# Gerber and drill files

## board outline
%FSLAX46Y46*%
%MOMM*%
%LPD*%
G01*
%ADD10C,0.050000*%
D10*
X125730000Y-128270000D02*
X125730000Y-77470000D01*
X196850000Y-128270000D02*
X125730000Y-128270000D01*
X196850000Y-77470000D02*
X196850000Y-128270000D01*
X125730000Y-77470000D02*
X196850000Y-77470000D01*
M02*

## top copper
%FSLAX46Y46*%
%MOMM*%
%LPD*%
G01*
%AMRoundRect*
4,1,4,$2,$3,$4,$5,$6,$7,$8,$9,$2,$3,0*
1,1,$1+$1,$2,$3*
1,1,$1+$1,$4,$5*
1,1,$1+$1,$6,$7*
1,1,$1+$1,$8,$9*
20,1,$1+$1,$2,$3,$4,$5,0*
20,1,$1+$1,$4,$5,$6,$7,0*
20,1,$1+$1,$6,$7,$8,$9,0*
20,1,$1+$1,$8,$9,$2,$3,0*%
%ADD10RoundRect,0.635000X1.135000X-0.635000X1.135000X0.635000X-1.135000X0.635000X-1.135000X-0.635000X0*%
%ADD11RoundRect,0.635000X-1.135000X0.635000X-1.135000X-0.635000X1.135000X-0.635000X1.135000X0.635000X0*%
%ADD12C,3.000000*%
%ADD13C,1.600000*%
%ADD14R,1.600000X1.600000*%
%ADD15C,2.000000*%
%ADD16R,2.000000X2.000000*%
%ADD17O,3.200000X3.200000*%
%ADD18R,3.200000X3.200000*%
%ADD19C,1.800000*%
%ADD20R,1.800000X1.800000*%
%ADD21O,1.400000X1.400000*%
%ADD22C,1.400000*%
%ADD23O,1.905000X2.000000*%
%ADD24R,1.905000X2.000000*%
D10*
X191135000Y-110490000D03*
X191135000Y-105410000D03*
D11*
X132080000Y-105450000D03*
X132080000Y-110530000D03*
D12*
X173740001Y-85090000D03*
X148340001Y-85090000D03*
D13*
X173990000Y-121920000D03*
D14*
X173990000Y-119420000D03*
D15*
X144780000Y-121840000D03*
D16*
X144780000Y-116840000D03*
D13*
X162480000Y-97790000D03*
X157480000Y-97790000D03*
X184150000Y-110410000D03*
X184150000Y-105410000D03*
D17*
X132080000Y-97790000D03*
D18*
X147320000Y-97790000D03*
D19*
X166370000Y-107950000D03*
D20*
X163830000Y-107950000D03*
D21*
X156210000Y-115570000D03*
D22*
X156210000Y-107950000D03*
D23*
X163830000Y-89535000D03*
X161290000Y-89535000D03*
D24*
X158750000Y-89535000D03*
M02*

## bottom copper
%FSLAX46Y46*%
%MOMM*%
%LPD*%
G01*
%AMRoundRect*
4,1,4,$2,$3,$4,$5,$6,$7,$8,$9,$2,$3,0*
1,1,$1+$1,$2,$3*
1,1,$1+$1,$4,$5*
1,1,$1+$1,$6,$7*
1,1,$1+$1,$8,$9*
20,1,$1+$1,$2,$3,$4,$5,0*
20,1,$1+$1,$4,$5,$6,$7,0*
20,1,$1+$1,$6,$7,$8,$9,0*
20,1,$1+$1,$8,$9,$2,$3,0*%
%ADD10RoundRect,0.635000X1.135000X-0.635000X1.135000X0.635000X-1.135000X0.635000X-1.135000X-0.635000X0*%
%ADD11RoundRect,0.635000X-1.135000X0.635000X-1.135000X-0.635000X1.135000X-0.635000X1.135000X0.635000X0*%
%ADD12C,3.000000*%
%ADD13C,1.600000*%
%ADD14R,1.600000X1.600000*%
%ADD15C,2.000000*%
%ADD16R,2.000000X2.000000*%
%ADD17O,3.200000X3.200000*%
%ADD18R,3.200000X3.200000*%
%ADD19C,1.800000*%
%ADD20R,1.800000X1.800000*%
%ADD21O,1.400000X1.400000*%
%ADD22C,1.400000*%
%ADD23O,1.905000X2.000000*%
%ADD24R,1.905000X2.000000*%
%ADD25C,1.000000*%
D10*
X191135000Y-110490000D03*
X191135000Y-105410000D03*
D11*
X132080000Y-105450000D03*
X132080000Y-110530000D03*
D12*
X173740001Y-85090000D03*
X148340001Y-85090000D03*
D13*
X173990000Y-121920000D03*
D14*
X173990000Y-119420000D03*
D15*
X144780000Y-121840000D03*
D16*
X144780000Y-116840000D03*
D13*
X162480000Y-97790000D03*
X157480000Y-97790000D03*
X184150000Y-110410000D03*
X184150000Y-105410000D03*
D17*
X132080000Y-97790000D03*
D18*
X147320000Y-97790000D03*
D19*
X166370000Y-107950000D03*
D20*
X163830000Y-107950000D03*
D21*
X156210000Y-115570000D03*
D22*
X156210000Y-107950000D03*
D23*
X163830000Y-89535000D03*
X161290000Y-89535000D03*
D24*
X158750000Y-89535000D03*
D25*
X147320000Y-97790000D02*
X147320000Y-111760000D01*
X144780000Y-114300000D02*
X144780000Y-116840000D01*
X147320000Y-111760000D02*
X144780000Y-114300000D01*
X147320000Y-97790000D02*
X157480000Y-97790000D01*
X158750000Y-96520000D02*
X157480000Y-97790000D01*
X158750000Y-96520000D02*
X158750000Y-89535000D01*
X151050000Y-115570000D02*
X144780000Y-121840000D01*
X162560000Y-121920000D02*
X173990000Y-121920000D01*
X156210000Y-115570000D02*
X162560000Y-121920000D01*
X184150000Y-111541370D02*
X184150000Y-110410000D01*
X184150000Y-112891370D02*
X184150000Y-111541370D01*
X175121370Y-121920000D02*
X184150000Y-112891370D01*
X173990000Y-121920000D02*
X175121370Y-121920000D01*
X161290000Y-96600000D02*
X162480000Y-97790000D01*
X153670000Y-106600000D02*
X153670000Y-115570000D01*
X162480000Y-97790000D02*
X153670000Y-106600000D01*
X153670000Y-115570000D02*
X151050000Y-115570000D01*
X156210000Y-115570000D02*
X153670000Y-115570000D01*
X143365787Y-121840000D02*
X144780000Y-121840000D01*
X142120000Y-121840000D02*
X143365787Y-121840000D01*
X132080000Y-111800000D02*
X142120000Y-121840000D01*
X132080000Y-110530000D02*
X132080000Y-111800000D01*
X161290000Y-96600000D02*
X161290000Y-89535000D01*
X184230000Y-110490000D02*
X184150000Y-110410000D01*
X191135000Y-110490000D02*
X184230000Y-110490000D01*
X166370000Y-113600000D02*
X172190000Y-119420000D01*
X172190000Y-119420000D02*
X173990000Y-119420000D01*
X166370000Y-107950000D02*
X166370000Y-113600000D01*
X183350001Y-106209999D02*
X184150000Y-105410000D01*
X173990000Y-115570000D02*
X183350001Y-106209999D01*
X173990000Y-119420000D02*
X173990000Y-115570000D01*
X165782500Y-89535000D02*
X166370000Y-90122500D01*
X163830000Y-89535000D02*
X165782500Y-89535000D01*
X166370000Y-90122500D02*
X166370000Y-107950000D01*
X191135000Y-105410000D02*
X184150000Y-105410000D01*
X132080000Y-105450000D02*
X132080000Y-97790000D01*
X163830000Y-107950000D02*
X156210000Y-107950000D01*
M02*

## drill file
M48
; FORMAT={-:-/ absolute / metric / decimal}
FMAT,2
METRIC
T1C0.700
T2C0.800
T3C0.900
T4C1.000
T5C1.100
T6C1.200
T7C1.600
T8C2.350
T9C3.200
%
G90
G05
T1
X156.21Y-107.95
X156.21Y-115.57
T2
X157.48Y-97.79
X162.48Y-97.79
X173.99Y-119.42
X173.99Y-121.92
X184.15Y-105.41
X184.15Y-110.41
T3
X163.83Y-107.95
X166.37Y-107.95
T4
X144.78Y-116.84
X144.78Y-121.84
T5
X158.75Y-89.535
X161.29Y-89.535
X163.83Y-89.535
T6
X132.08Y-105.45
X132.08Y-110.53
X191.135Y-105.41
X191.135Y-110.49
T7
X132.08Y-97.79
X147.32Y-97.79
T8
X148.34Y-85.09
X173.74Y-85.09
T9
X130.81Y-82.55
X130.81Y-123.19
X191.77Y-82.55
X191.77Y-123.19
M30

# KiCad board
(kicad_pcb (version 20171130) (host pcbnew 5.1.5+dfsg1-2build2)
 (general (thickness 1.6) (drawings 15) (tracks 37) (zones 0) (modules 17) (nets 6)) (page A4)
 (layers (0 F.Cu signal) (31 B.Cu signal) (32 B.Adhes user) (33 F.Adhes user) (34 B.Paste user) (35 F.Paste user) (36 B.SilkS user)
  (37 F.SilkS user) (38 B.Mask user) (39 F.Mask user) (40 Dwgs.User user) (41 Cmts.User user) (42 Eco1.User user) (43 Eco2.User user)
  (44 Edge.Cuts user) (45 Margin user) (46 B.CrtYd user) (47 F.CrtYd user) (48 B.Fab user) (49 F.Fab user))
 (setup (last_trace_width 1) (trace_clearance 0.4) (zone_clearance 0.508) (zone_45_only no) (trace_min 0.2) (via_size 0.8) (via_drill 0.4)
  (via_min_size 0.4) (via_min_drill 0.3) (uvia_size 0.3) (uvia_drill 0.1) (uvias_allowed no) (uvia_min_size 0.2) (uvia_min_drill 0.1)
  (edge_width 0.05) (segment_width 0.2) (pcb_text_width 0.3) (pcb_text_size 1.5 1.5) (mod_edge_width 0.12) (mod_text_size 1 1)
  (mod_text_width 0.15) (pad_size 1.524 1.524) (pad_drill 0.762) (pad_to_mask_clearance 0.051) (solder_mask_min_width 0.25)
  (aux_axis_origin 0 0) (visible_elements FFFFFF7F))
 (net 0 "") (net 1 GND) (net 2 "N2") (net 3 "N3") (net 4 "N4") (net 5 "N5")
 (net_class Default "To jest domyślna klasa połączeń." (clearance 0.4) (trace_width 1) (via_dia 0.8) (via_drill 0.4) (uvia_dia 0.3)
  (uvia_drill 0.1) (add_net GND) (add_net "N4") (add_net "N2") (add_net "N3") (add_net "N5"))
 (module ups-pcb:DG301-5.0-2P (layer F.Cu) (at 191.135 107.99 90)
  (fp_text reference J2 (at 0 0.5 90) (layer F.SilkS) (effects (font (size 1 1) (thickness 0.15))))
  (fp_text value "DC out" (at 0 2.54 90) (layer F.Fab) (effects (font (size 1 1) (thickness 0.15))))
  (pad 1 thru_hole roundrect (at -2.5 0 90) (size 2.54 3.54) (drill 1.2) (layers *.Cu *.Mask) (roundrect_rratio 0.25) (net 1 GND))
  (pad 2 thru_hole roundrect (at 2.58 0 90) (size 2.54 3.54) (drill 1.2) (layers *.Cu *.Mask) (roundrect_rratio 0.25) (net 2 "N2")))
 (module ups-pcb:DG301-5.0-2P (layer F.Cu) (at 132.08 107.95 270)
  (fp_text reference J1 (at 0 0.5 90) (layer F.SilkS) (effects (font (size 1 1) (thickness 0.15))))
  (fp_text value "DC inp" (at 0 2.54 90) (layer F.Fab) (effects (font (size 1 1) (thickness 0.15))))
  (pad 1 thru_hole roundrect (at -2.5 0 270) (size 2.54 3.54) (drill 1.2) (layers *.Cu *.Mask) (roundrect_rratio 0.25) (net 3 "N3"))
  (pad 2 thru_hole roundrect (at 2.58 0 270) (size 2.54 3.54) (drill 1.2) (layers *.Cu *.Mask) (roundrect_rratio 0.25) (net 1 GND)))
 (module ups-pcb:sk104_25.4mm (layer F.Cu) (at 161.040001 85.09)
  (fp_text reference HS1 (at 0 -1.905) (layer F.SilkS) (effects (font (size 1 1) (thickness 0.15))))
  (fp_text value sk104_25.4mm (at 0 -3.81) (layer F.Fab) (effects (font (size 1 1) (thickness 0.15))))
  (pad "" np_thru_hole circle (at 12.7 0) (size 3 3) (drill 2.35) (layers *.Cu *.Mask))
  (pad "" np_thru_hole circle (at -12.7 0) (size 3 3) (drill 2.35) (layers *.Cu *.Mask)))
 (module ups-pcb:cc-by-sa (layer F.Cu) (at 159.385 121.92)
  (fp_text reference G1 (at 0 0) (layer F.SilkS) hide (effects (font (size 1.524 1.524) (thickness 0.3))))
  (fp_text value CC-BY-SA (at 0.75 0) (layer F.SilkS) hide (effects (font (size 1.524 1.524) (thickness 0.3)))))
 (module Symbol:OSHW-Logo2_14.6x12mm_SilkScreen (layer F.Cu) (at 186.055 93.98)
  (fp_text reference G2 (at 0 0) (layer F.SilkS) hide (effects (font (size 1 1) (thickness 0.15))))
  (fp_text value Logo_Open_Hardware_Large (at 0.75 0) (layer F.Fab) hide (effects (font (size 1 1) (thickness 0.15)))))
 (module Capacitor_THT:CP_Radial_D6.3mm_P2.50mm (layer F.Cu) (at 173.99 119.42 270)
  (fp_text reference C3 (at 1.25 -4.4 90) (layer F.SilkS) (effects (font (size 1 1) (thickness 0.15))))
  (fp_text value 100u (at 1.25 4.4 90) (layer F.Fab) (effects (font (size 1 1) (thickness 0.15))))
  (pad 2 thru_hole circle (at 2.5 0 270) (size 1.6 1.6) (drill 0.8) (layers *.Cu *.Mask) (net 1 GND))
  (pad 1 thru_hole rect (at 0 0 270) (size 1.6 1.6) (drill 0.8) (layers *.Cu *.Mask) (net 2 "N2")))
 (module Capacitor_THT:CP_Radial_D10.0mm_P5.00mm (layer F.Cu) (at 144.78 116.84 270)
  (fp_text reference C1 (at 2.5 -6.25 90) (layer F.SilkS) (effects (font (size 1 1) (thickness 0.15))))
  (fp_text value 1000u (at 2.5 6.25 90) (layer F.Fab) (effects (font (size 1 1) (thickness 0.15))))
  (pad 2 thru_hole circle (at 5 0 270) (size 2 2) (drill 1) (layers *.Cu *.Mask) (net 1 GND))
  (pad 1 thru_hole rect (at 0 0 270) (size 2 2) (drill 1) (layers *.Cu *.Mask) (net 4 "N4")))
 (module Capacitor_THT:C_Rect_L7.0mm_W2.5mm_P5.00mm (layer F.Cu) (at 157.48 97.79)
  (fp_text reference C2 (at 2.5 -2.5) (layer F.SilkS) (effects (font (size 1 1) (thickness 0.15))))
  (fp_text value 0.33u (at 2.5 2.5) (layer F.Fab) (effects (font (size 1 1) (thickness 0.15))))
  (pad 2 thru_hole circle (at 5 0) (size 1.6 1.6) (drill 0.8) (layers *.Cu *.Mask) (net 1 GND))
  (pad 1 thru_hole circle (at 0 0) (size 1.6 1.6) (drill 0.8) (layers *.Cu *.Mask) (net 4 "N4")))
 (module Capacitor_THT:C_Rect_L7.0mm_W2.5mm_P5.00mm (layer F.Cu) (at 184.15 105.41 270)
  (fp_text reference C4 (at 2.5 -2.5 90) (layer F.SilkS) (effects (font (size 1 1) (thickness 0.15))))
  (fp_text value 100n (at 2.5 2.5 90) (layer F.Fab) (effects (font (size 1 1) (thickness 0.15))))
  (pad 2 thru_hole circle (at 5 0 270) (size 1.6 1.6) (drill 0.8) (layers *.Cu *.Mask) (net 1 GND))
  (pad 1 thru_hole circle (at 0 0 270) (size 1.6 1.6) (drill 0.8) (layers *.Cu *.Mask) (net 2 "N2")))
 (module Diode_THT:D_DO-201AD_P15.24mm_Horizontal (layer F.Cu) (at 147.32 97.79 180)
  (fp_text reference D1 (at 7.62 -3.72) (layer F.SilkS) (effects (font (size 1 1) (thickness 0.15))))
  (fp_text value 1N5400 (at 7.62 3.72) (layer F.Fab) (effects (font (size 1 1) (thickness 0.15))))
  (pad 2 thru_hole oval (at 15.24 0 180) (size 3.2 3.2) (drill 1.6) (layers *.Cu *.Mask) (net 3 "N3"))
  (pad 1 thru_hole rect (at 0 0 180) (size 3.2 3.2) (drill 1.6) (layers *.Cu *.Mask) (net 4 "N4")))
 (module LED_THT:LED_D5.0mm (layer F.Cu) (at 163.83 107.95)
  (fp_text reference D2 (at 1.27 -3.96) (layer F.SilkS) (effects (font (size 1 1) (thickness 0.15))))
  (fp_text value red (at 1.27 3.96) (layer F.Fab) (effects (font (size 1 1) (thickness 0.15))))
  (pad 2 thru_hole circle (at 2.54 0) (size 1.8 1.8) (drill 0.9) (layers *.Cu *.Mask) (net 2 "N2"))
  (pad 1 thru_hole rect (at 0 0) (size 1.8 1.8) (drill 0.9) (layers *.Cu *.Mask) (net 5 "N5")))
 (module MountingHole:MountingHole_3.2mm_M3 (layer F.Cu) (at 130.81 82.55)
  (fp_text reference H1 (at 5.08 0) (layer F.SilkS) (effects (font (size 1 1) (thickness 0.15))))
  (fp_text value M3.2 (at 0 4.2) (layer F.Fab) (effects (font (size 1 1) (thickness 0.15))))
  (pad 1 np_thru_hole circle (at 0 0) (size 3.2 3.2) (drill 3.2) (layers *.Cu *.Mask)))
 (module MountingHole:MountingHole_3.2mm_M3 (layer F.Cu) (at 191.77 82.55)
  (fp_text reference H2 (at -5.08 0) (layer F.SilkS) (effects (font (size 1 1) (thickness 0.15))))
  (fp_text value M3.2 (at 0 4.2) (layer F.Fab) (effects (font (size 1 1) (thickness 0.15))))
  (pad 1 np_thru_hole circle (at 0 0) (size 3.2 3.2) (drill 3.2) (layers *.Cu *.Mask)))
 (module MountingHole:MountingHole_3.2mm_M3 (layer F.Cu) (at 191.77 123.19)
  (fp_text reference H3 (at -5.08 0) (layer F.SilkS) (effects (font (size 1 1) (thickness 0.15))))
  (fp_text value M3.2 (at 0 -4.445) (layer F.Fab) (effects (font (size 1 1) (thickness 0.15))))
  (pad 1 np_thru_hole circle (at 0 0) (size 3.2 3.2) (drill 3.2) (layers *.Cu *.Mask)))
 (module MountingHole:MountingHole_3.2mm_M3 (layer F.Cu) (at 130.81 123.19)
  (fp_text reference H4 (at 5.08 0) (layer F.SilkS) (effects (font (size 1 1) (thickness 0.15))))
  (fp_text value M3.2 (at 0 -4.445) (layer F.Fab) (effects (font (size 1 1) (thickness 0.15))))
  (pad 1 np_thru_hole circle (at 0 0) (size 3.2 3.2) (drill 3.2) (layers *.Cu *.Mask)))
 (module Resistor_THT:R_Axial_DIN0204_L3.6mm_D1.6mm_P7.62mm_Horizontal (layer F.Cu) (at 156.21 107.95 270)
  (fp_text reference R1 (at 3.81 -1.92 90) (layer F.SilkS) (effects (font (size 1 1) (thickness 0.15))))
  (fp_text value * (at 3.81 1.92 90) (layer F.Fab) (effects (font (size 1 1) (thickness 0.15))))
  (pad 2 thru_hole oval (at 7.62 0 270) (size 1.4 1.4) (drill 0.7) (layers *.Cu *.Mask) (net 1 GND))
  (pad 1 thru_hole circle (at 0 0 270) (size 1.4 1.4) (drill 0.7) (layers *.Cu *.Mask) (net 5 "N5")))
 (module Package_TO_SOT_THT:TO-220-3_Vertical (layer F.Cu) (at 158.75 89.535)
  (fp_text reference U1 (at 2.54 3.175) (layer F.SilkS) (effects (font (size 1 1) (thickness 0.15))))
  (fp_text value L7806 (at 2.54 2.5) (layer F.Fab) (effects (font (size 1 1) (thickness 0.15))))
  (pad 3 thru_hole oval (at 5.08 0) (size 1.905 2) (drill 1.1) (layers *.Cu *.Mask) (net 2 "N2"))
  (pad 2 thru_hole oval (at 2.54 0) (size 1.905 2) (drill 1.1) (layers *.Cu *.Mask) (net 1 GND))
  (pad 1 thru_hole rect (at 0 0) (size 1.905 2) (drill 1.1) (layers *.Cu *.Mask) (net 4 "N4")))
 (gr_line (start 125.73 128.27) (end 125.73 77.47) (layer Edge.Cuts) (width 0.05))
 (gr_line (start 196.85 128.27) (end 125.73 128.27) (layer Edge.Cuts) (width 0.05))
 (gr_line (start 196.85 77.47) (end 196.85 128.27) (layer Edge.Cuts) (width 0.05))
 (gr_line (start 125.73 77.47) (end 196.85 77.47) (layer Edge.Cuts) (width 0.05))
 (segment (start 147.32 97.79) (end 147.32 111.76) (width 1) (layer B.Cu) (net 4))
 (segment (start 144.78 114.3) (end 144.78 116.84) (width 1) (layer B.Cu) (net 4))
 (segment (start 147.32 111.76) (end 144.78 114.3) (width 1) (layer B.Cu) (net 4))
 (segment (start 147.32 97.79) (end 157.48 97.79) (width 1) (layer B.Cu) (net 4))
 (segment (start 158.75 96.52) (end 157.48 97.79) (width 1) (layer B.Cu) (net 4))
 (segment (start 158.75 96.52) (end 158.75 89.535) (width 1) (layer B.Cu) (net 4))
 (segment (start 151.05 115.57) (end 144.78 121.84) (width 1) (layer B.Cu) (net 1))
 (segment (start 162.56 121.92) (end 173.99 121.92) (width 1) (layer B.Cu) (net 1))
 (segment (start 156.21 115.57) (end 162.56 121.92) (width 1) (layer B.Cu) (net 1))
 (segment (start 184.15 111.54137) (end 184.15 110.41) (width 1) (layer B.Cu) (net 1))
 (segment (start 184.15 112.89137) (end 184.15 111.54137) (width 1) (layer B.Cu) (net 1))
 (segment (start 175.12137 121.92) (end 184.15 112.89137) (width 1) (layer B.Cu) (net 1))
 (segment (start 173.99 121.92) (end 175.12137 121.92) (width 1) (layer B.Cu) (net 1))
 (segment (start 161.29 96.6) (end 162.48 97.79) (width 1) (layer B.Cu) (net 1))
 (segment (start 153.67 106.6) (end 153.67 115.57) (width 1) (layer B.Cu) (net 1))
 (segment (start 162.48 97.79) (end 153.67 106.6) (width 1) (layer B.Cu) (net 1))
 (segment (start 153.67 115.57) (end 151.05 115.57) (width 1) (layer B.Cu) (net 1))
 (segment (start 156.21 115.57) (end 153.67 115.57) (width 1) (layer B.Cu) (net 1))
 (segment (start 143.365787 121.84) (end 144.78 121.84) (width 1) (layer B.Cu) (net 1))
 (segment (start 142.12 121.84) (end 143.365787 121.84) (width 1) (layer B.Cu) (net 1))
 (segment (start 132.08 111.8) (end 142.12 121.84) (width 1) (layer B.Cu) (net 1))
 (segment (start 132.08 110.53) (end 132.08 111.8) (width 1) (layer B.Cu) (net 1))
 (segment (start 161.29 96.6) (end 161.29 89.535) (width 1) (layer B.Cu) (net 1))
 (segment (start 184.23 110.49) (end 184.15 110.41) (width 1) (layer B.Cu) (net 1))
 (segment (start 191.135 110.49) (end 184.23 110.49) (width 1) (layer B.Cu) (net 1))
 (segment (start 166.37 113.6) (end 172.19 119.42) (width 1) (layer B.Cu) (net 2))
 (segment (start 172.19 119.42) (end 173.99 119.42) (width 1) (layer B.Cu) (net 2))
 (segment (start 166.37 107.95) (end 166.37 113.6) (width 1) (layer B.Cu) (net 2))
 (segment (start 183.350001 106.209999) (end 184.15 105.41) (width 1) (layer B.Cu) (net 2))
 (segment (start 173.99 115.57) (end 183.350001 106.209999) (width 1) (layer B.Cu) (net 2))
 (segment (start 173.99 119.42) (end 173.99 115.57) (width 1) (layer B.Cu) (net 2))
 (segment (start 165.7825 89.535) (end 166.37 90.1225) (width 1) (layer B.Cu) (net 2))
 (segment (start 163.83 89.535) (end 165.7825 89.535) (width 1) (layer B.Cu) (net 2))
 (segment (start 166.37 90.1225) (end 166.37 107.95) (width 1) (layer B.Cu) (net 2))
 (segment (start 191.135 105.41) (end 184.15 105.41) (width 1) (layer B.Cu) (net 2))
 (segment (start 132.08 105.45) (end 132.08 97.79) (width 1) (layer B.Cu) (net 3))
 (segment (start 163.83 107.95) (end 156.21 107.95) (width 1) (layer B.Cu) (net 5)))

